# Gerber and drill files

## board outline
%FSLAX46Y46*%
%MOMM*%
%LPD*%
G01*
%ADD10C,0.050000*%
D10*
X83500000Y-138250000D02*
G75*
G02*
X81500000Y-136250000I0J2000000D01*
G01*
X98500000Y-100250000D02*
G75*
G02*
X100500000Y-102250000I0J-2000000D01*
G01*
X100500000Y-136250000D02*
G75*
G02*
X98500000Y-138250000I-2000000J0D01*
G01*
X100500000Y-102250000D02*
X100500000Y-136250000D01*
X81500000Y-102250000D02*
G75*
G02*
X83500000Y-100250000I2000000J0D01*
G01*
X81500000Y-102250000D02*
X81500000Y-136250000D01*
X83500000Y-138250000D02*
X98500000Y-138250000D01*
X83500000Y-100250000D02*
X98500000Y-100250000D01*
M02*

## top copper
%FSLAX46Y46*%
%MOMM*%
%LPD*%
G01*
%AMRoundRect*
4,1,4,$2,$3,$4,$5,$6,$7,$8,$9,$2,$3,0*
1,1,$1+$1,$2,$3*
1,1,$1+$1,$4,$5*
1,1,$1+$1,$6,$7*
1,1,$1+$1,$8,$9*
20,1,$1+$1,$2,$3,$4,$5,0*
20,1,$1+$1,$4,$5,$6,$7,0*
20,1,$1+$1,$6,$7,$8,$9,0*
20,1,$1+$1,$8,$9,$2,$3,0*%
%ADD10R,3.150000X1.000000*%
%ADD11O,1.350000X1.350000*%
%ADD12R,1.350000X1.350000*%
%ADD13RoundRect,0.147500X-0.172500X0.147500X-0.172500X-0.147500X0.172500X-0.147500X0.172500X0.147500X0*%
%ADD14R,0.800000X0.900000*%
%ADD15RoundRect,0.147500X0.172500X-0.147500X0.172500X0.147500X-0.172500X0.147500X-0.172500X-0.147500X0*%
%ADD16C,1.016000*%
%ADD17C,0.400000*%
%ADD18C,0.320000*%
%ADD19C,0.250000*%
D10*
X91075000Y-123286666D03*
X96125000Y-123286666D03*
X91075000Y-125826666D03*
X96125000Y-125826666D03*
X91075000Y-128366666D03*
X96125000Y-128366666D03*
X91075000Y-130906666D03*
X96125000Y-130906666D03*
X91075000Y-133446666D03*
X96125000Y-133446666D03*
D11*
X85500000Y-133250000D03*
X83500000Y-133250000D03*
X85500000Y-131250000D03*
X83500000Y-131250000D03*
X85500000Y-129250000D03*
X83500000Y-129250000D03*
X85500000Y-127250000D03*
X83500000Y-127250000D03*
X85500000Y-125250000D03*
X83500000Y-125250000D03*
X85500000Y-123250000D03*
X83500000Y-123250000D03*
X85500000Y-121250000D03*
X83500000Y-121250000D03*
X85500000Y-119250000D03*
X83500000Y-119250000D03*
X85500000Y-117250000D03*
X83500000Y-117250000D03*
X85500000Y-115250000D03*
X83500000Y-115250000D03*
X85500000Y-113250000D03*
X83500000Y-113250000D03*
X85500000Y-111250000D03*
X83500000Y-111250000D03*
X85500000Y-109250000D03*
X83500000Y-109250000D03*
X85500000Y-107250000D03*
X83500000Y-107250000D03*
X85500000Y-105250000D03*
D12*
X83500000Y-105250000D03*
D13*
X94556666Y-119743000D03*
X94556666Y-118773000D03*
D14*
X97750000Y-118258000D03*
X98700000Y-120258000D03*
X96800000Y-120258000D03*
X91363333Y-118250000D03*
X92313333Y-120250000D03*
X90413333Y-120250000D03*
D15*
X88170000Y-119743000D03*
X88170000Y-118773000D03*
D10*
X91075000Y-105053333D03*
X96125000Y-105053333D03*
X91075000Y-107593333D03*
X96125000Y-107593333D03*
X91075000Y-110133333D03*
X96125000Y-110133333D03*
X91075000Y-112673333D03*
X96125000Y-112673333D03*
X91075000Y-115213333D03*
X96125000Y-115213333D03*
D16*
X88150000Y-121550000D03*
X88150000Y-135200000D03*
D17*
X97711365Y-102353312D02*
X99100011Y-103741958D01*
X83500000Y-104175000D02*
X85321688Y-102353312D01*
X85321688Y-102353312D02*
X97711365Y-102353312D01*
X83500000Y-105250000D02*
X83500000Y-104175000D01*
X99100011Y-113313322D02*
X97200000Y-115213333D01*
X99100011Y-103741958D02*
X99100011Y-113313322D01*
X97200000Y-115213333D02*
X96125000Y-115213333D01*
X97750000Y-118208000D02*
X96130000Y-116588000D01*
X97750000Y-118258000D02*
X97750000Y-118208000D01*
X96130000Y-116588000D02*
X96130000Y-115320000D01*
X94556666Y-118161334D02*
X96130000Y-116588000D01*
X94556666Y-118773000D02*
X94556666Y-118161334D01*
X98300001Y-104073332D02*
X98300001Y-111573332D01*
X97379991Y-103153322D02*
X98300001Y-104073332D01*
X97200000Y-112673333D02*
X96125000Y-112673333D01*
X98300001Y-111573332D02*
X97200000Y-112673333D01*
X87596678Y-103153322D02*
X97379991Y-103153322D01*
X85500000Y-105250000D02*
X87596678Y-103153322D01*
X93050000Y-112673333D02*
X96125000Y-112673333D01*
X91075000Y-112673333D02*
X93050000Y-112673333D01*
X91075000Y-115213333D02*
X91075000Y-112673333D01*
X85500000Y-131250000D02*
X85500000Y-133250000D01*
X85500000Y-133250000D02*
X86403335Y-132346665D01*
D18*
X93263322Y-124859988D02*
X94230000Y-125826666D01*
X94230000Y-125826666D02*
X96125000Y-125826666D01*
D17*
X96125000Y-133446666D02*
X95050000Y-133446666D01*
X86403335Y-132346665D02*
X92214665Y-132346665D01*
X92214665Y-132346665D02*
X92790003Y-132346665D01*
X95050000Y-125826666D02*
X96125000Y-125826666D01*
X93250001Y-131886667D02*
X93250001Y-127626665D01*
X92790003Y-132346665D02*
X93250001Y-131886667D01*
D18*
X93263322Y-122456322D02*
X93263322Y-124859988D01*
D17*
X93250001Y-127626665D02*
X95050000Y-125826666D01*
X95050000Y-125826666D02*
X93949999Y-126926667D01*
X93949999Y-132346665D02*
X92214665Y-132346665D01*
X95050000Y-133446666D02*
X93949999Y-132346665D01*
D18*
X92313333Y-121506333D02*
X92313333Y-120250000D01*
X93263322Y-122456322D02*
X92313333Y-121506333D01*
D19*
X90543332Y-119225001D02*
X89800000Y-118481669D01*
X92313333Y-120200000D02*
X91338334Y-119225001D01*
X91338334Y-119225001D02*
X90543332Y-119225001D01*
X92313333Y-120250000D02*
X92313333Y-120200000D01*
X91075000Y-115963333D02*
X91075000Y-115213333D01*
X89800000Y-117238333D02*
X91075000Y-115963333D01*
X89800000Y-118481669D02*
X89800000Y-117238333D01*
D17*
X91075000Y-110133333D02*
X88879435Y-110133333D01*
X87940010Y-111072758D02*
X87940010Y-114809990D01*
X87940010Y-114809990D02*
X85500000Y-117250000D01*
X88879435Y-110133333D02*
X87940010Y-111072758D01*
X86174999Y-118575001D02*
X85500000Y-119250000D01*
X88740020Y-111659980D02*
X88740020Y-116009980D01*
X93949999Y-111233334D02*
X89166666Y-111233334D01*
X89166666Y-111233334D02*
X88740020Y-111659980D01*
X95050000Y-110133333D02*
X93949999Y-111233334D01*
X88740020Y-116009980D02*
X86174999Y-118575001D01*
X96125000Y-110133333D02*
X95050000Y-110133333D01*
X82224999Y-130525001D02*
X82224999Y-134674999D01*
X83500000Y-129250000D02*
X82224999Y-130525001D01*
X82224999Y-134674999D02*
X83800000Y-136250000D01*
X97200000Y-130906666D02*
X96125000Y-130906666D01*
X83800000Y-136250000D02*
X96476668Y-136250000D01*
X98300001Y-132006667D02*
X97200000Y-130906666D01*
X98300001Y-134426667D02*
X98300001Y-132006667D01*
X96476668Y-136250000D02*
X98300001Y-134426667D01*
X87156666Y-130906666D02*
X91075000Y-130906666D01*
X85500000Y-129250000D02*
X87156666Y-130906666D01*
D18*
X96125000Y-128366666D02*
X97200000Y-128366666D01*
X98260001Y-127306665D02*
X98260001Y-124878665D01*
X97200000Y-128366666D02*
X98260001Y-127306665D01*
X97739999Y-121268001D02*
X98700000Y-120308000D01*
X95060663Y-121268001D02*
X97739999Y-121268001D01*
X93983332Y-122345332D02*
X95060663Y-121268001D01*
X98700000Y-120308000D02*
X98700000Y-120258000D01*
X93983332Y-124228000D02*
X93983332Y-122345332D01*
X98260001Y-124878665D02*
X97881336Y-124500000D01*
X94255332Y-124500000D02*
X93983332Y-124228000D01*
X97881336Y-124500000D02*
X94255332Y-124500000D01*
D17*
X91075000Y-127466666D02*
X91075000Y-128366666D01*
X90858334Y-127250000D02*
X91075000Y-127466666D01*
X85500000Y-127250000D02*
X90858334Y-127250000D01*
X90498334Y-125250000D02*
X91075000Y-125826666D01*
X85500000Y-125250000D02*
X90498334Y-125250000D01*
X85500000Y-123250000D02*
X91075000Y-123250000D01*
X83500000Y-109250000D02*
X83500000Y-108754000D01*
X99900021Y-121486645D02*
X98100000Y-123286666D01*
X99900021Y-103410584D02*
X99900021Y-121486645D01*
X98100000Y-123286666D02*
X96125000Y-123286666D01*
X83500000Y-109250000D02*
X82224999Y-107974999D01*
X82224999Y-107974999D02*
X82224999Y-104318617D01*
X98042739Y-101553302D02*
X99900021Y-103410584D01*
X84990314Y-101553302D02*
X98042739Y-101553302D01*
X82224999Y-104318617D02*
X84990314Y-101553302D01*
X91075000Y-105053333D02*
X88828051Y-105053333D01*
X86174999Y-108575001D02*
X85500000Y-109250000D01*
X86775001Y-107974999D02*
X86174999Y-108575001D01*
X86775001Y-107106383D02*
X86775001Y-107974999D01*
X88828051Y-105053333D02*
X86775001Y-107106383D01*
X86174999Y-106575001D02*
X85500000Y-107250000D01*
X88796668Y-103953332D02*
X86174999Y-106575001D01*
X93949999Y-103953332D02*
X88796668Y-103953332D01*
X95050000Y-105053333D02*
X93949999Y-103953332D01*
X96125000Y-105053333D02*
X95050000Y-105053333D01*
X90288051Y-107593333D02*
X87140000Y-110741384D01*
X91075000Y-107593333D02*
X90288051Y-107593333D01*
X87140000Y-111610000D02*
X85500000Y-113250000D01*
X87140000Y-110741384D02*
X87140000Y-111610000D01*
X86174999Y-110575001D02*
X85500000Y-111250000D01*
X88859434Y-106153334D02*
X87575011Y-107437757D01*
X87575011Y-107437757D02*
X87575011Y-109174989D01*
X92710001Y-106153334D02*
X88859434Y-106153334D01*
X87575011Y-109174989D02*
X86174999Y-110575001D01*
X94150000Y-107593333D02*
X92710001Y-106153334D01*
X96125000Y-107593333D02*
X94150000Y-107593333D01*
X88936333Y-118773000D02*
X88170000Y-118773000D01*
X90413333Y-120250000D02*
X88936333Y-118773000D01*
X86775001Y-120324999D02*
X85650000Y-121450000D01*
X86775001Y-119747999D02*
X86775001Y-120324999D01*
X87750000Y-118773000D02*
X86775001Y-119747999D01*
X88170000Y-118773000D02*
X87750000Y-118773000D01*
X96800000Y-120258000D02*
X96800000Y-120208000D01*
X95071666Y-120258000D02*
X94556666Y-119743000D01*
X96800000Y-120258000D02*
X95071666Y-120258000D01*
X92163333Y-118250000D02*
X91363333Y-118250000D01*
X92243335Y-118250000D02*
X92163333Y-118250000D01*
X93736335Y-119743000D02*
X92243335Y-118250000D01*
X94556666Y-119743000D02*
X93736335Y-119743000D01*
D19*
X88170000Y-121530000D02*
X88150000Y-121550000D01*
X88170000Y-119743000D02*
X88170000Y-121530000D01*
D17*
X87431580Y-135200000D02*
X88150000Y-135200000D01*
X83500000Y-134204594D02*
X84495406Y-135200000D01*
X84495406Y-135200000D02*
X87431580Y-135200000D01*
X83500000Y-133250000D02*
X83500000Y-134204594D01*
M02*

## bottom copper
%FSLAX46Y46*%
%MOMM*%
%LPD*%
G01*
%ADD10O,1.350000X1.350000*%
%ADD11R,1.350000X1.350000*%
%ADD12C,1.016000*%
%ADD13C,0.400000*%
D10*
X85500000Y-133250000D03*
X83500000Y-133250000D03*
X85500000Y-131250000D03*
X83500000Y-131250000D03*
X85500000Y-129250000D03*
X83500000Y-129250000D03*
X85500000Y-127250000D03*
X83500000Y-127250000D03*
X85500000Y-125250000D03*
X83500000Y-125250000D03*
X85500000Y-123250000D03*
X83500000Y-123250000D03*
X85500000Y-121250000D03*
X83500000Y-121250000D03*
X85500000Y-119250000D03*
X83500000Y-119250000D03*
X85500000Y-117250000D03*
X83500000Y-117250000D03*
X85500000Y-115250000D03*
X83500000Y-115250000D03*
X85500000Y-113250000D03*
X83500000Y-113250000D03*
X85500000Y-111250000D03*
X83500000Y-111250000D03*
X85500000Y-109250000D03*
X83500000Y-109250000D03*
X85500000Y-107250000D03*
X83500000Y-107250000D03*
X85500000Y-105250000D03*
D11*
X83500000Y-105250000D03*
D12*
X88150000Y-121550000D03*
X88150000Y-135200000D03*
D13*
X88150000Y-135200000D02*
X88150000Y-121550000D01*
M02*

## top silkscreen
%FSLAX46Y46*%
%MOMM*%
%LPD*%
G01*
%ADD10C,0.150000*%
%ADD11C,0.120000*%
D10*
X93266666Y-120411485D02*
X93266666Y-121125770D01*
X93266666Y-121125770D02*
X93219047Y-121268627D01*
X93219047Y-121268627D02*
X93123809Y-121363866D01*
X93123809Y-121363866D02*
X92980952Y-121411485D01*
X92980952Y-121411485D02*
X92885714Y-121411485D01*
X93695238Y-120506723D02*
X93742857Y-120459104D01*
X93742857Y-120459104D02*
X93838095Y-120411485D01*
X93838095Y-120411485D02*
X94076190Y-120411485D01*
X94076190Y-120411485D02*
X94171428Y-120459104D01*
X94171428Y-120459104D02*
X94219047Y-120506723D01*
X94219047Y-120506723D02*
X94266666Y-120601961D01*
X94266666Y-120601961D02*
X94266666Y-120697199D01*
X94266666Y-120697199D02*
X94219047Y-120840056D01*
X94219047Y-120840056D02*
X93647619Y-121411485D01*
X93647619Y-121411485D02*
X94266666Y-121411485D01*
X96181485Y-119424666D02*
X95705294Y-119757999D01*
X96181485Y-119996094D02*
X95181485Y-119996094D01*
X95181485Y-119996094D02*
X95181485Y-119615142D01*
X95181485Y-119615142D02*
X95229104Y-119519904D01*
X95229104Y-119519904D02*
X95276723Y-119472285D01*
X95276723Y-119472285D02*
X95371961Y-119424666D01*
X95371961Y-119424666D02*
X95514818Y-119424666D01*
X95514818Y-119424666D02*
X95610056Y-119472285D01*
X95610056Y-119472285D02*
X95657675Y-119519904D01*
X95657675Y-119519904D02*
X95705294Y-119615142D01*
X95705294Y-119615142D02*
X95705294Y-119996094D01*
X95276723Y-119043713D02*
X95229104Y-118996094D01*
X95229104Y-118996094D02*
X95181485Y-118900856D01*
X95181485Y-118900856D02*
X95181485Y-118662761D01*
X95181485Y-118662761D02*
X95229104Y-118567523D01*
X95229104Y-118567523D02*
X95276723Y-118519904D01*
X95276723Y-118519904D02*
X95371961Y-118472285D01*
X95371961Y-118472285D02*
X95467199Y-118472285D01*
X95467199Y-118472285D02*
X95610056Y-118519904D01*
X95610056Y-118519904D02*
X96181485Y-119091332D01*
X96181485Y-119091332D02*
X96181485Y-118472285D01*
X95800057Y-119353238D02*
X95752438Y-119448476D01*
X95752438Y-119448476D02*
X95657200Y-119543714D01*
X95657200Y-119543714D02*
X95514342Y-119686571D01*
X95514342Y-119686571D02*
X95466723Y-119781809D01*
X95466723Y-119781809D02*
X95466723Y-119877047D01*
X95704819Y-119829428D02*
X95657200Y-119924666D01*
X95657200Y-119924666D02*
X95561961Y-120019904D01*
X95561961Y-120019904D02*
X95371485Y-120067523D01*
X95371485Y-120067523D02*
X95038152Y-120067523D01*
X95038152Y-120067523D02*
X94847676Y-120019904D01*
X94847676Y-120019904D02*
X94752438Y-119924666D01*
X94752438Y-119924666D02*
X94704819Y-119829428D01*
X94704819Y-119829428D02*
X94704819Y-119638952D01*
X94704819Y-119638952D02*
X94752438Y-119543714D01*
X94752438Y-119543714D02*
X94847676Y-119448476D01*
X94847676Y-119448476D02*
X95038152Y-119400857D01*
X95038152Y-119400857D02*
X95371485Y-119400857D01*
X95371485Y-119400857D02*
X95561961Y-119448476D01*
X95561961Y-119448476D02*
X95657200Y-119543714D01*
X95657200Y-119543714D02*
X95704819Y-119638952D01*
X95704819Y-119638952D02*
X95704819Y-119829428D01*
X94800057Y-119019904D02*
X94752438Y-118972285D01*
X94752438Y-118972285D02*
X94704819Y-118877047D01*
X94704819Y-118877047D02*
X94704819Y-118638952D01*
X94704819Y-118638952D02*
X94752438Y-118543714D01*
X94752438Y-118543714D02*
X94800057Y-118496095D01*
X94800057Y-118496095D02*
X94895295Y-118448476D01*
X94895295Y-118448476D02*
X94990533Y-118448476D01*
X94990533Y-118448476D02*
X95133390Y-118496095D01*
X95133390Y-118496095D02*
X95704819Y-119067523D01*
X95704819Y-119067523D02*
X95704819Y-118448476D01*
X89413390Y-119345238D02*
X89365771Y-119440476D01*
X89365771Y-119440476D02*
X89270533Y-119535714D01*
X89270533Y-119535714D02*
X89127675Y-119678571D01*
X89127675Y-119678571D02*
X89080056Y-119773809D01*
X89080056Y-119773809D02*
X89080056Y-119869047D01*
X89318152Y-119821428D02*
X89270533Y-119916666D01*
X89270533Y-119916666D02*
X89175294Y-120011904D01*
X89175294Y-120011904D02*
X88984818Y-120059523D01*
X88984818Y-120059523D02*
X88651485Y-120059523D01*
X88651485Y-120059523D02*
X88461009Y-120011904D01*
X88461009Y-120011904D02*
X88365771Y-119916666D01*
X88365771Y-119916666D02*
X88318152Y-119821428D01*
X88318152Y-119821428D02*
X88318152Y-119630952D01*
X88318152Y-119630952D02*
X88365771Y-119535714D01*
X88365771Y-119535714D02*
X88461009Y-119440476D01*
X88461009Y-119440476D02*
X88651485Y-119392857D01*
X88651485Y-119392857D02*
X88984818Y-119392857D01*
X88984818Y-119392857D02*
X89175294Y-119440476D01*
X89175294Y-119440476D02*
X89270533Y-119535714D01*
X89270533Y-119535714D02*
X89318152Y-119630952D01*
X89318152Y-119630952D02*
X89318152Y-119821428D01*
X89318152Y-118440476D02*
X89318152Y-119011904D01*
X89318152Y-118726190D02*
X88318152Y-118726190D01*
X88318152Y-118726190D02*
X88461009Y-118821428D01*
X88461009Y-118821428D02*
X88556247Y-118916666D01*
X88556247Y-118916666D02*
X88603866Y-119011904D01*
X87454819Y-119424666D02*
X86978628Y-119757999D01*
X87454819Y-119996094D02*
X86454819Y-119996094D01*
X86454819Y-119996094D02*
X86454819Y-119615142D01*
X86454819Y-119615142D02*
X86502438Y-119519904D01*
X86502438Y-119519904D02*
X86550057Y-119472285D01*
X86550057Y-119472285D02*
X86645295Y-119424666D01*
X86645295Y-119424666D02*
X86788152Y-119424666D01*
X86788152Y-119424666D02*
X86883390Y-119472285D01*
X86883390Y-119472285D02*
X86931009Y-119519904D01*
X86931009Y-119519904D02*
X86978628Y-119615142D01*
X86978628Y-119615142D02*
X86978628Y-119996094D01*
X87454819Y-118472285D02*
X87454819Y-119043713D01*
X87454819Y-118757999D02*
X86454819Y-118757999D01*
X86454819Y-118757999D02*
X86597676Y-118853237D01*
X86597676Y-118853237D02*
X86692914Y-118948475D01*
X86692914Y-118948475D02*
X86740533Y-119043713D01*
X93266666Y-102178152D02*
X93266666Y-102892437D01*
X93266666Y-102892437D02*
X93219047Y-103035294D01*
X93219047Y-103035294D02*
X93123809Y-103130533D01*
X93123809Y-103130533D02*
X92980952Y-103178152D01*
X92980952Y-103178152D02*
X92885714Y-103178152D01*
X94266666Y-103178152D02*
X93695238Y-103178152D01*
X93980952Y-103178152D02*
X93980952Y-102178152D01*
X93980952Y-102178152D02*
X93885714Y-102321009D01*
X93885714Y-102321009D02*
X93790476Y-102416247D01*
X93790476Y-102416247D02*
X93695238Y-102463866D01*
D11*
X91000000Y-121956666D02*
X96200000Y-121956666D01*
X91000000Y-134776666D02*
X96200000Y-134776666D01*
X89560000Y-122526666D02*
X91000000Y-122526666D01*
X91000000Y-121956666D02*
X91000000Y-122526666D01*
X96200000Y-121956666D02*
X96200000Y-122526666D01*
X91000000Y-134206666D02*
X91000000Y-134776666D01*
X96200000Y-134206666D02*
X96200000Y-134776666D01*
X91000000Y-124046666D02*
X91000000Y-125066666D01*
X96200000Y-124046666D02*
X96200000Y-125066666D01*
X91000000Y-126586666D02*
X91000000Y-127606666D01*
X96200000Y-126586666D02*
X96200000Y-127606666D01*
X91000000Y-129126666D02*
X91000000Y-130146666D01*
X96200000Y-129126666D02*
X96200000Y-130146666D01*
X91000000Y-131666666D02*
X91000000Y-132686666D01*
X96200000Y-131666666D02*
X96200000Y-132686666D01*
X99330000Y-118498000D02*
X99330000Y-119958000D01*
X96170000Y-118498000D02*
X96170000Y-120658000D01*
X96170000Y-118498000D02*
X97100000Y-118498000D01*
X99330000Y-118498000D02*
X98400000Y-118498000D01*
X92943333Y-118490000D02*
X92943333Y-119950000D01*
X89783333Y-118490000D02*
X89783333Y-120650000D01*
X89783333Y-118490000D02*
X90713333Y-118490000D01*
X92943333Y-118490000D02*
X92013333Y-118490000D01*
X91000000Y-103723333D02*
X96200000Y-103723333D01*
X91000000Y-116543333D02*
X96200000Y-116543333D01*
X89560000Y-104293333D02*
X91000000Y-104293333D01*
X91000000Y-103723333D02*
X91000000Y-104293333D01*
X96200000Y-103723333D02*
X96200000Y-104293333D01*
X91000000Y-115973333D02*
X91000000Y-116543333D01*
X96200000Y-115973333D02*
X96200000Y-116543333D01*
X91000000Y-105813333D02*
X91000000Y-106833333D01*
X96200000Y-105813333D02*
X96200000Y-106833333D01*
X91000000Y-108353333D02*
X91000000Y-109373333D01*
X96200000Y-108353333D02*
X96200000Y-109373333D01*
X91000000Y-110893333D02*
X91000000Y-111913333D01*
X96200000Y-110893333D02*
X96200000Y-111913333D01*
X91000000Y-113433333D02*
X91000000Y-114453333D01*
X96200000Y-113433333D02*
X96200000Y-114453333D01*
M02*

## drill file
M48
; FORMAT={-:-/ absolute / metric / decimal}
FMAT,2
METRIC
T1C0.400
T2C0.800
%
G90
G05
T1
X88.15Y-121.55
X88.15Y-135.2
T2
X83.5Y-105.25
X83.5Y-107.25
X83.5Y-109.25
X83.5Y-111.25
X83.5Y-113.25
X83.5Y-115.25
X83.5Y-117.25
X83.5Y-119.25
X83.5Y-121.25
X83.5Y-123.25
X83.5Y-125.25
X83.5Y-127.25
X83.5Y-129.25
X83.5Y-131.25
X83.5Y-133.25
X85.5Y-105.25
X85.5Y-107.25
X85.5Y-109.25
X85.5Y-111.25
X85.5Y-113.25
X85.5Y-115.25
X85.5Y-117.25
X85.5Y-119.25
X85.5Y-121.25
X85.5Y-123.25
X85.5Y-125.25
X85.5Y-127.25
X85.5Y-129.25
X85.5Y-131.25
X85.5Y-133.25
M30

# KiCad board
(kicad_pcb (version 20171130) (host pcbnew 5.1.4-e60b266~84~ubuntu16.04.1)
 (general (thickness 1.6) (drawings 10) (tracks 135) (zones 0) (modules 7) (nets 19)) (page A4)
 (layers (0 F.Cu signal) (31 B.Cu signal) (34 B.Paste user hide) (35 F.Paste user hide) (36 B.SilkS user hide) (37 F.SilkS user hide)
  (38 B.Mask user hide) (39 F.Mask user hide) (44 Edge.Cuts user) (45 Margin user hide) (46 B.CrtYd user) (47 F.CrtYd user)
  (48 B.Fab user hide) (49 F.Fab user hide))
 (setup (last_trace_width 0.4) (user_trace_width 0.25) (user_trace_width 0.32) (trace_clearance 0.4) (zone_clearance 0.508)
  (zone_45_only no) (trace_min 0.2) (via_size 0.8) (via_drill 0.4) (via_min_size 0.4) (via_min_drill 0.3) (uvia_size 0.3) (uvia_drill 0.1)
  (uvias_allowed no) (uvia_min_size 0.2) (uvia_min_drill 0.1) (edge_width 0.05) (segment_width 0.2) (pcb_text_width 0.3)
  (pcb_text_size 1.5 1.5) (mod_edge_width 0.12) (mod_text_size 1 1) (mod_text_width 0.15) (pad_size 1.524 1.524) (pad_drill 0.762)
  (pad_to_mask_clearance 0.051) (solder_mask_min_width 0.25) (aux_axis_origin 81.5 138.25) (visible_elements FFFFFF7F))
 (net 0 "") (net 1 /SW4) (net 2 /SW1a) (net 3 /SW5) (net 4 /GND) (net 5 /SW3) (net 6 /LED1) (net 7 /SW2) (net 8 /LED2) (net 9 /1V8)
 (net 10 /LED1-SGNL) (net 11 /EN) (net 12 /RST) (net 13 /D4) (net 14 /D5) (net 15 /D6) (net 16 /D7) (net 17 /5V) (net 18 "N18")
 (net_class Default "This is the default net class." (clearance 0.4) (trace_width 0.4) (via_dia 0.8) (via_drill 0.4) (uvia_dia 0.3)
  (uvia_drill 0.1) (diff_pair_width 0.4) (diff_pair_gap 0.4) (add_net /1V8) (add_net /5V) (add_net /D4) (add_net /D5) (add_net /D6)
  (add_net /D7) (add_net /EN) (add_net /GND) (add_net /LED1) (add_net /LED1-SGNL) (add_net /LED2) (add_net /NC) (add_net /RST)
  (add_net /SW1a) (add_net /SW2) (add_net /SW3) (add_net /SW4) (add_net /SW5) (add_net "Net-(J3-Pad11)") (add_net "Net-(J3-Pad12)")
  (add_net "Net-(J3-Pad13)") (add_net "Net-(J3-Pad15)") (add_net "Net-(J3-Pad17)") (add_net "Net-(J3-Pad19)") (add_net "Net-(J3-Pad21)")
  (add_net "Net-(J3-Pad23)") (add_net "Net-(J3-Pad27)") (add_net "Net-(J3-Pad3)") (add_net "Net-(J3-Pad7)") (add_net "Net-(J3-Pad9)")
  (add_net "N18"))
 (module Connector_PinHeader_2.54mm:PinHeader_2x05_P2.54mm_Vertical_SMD (layer F.Cu) (at 93.6 128.366666)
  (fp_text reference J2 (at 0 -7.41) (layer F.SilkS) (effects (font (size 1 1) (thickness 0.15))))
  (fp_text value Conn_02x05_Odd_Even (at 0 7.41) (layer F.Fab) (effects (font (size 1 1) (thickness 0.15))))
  (fp_line (start -2.6 -6.41) (end 2.6 -6.41) (layer F.SilkS) (width 0.12))
  (fp_line (start -2.6 6.41) (end 2.6 6.41) (layer F.SilkS) (width 0.12))
  (fp_line (start -4.04 -5.84) (end -2.6 -5.84) (layer F.SilkS) (width 0.12))
  (fp_line (start -2.6 -6.41) (end -2.6 -5.84) (layer F.SilkS) (width 0.12))
  (fp_line (start 2.6 -6.41) (end 2.6 -5.84) (layer F.SilkS) (width 0.12))
  (fp_line (start -2.6 5.84) (end -2.6 6.41) (layer F.SilkS) (width 0.12))
  (fp_line (start 2.6 5.84) (end 2.6 6.41) (layer F.SilkS) (width 0.12))
  (fp_line (start -2.6 -4.32) (end -2.6 -3.3) (layer F.SilkS) (width 0.12))
  (fp_line (start 2.6 -4.32) (end 2.6 -3.3) (layer F.SilkS) (width 0.12))
  (fp_line (start -2.6 -1.78) (end -2.6 -0.76) (layer F.SilkS) (width 0.12))
  (fp_line (start 2.6 -1.78) (end 2.6 -0.76) (layer F.SilkS) (width 0.12))
  (fp_line (start -2.6 0.76) (end -2.6 1.78) (layer F.SilkS) (width 0.12))
  (fp_line (start 2.6 0.76) (end 2.6 1.78) (layer F.SilkS) (width 0.12))
  (fp_line (start -2.6 3.3) (end -2.6 4.32) (layer F.SilkS) (width 0.12))
  (fp_line (start 2.6 3.3) (end 2.6 4.32) (layer F.SilkS) (width 0.12))
  (pad 1 smd rect (at -2.525 -5.08) (size 3.15 1) (layers F.Cu F.Paste F.Mask) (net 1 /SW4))
  (pad 2 smd rect (at 2.525 -5.08) (size 3.15 1) (layers F.Cu F.Paste F.Mask) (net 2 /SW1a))
  (pad 3 smd rect (at -2.525 -2.54) (size 3.15 1) (layers F.Cu F.Paste F.Mask) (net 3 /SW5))
  (pad 4 smd rect (at 2.525 -2.54) (size 3.15 1) (layers F.Cu F.Paste F.Mask) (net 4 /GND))
  (pad 5 smd rect (at -2.525 0) (size 3.15 1) (layers F.Cu F.Paste F.Mask) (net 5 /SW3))
  (pad 6 smd rect (at 2.525 0) (size 3.15 1) (layers F.Cu F.Paste F.Mask) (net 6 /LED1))
  (pad 7 smd rect (at -2.525 2.54) (size 3.15 1) (layers F.Cu F.Paste F.Mask) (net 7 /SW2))
  (pad 8 smd rect (at 2.525 2.54) (size 3.15 1) (layers F.Cu F.Paste F.Mask) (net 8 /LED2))
  (pad 9 smd rect (at -2.525 5.08) (size 3.15 1) (layers F.Cu F.Paste F.Mask))
  (pad 10 smd rect (at 2.525 5.08) (size 3.15 1) (layers F.Cu F.Paste F.Mask) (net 4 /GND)))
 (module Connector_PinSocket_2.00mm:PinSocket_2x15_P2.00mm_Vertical (layer B.Cu) (at 83.5 105.25 180)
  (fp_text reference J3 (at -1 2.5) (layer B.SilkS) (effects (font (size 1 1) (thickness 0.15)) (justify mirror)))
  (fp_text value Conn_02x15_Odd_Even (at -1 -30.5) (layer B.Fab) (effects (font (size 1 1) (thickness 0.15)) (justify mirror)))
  (pad 30 thru_hole oval (at -2 -28 180) (size 1.35 1.35) (drill 0.8) (layers *.Cu *.Mask) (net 4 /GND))
  (pad 29 thru_hole oval (at 0 -28 180) (size 1.35 1.35) (drill 0.8) (layers *.Cu *.Mask) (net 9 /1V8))
  (pad 28 thru_hole oval (at -2 -26 180) (size 1.35 1.35) (drill 0.8) (layers *.Cu *.Mask) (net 4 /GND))
  (pad 27 thru_hole oval (at 0 -26 180) (size 1.35 1.35) (drill 0.8) (layers *.Cu *.Mask))
  (pad 26 thru_hole oval (at -2 -24 180) (size 1.35 1.35) (drill 0.8) (layers *.Cu *.Mask) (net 7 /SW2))
  (pad 25 thru_hole oval (at 0 -24 180) (size 1.35 1.35) (drill 0.8) (layers *.Cu *.Mask) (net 8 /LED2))
  (pad 24 thru_hole oval (at -2 -22 180) (size 1.35 1.35) (drill 0.8) (layers *.Cu *.Mask) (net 5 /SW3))
  (pad 23 thru_hole oval (at 0 -22 180) (size 1.35 1.35) (drill 0.8) (layers *.Cu *.Mask))
  (pad 22 thru_hole oval (at -2 -20 180) (size 1.35 1.35) (drill 0.8) (layers *.Cu *.Mask) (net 3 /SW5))
  (pad 21 thru_hole oval (at 0 -20 180) (size 1.35 1.35) (drill 0.8) (layers *.Cu *.Mask))
  (pad 20 thru_hole oval (at -2 -18 180) (size 1.35 1.35) (drill 0.8) (layers *.Cu *.Mask) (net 1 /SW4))
  (pad 19 thru_hole oval (at 0 -18 180) (size 1.35 1.35) (drill 0.8) (layers *.Cu *.Mask))
  (pad 18 thru_hole oval (at -2 -16 180) (size 1.35 1.35) (drill 0.8) (layers *.Cu *.Mask) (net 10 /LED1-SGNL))
  (pad 17 thru_hole oval (at 0 -16 180) (size 1.35 1.35) (drill 0.8) (layers *.Cu *.Mask))
  (pad 16 thru_hole oval (at -2 -14 180) (size 1.35 1.35) (drill 0.8) (layers *.Cu *.Mask) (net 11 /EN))
  (pad 15 thru_hole oval (at 0 -14 180) (size 1.35 1.35) (drill 0.8) (layers *.Cu *.Mask))
  (pad 14 thru_hole oval (at -2 -12 180) (size 1.35 1.35) (drill 0.8) (layers *.Cu *.Mask) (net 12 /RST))
  (pad 13 thru_hole oval (at 0 -12 180) (size 1.35 1.35) (drill 0.8) (layers *.Cu *.Mask))
  (pad 12 thru_hole oval (at -2 -10 180) (size 1.35 1.35) (drill 0.8) (layers *.Cu *.Mask))
  (pad 11 thru_hole oval (at 0 -10 180) (size 1.35 1.35) (drill 0.8) (layers *.Cu *.Mask))
  (pad 10 thru_hole oval (at -2 -8 180) (size 1.35 1.35) (drill 0.8) (layers *.Cu *.Mask) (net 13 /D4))
  (pad 9 thru_hole oval (at 0 -8 180) (size 1.35 1.35) (drill 0.8) (layers *.Cu *.Mask))
  (pad 8 thru_hole oval (at -2 -6 180) (size 1.35 1.35) (drill 0.8) (layers *.Cu *.Mask) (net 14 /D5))
  (pad 7 thru_hole oval (at 0 -6 180) (size 1.35 1.35) (drill 0.8) (layers *.Cu *.Mask))
  (pad 6 thru_hole oval (at -2 -4 180) (size 1.35 1.35) (drill 0.8) (layers *.Cu *.Mask) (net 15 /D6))
  (pad 5 thru_hole oval (at 0 -4 180) (size 1.35 1.35) (drill 0.8) (layers *.Cu *.Mask) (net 2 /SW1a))
  (pad 4 thru_hole oval (at -2 -2 180) (size 1.35 1.35) (drill 0.8) (layers *.Cu *.Mask) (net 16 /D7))
  (pad 3 thru_hole oval (at 0 -2 180) (size 1.35 1.35) (drill 0.8) (layers *.Cu *.Mask))
  (pad 2 thru_hole oval (at -2 0 180) (size 1.35 1.35) (drill 0.8) (layers *.Cu *.Mask) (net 4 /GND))
  (pad 1 thru_hole rect (at 0 0 180) (size 1.35 1.35) (drill 0.8) (layers *.Cu *.Mask) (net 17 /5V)))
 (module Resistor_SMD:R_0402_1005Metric (layer F.Cu) (at 94.556666 119.258 270)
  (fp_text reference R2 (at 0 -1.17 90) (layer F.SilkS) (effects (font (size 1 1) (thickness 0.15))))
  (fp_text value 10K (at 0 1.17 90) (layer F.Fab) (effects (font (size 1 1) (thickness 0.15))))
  (pad 2 smd roundrect (at 0.485 0 270) (size 0.59 0.64) (layers F.Cu F.Paste F.Mask) (roundrect_rratio 0.25) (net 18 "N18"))
  (pad 1 smd roundrect (at -0.485 0 270) (size 0.59 0.64) (layers F.Cu F.Paste F.Mask) (roundrect_rratio 0.25) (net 17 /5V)))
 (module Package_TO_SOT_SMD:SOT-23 (layer F.Cu) (at 97.75 119.258 90)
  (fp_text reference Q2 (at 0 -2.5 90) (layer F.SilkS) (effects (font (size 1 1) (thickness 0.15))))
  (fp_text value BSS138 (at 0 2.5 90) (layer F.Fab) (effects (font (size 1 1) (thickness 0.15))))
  (fp_line (start 0.76 1.58) (end -0.7 1.58) (layer F.SilkS) (width 0.12))
  (fp_line (start 0.76 -1.58) (end -1.4 -1.58) (layer F.SilkS) (width 0.12))
  (fp_line (start 0.76 -1.58) (end 0.76 -0.65) (layer F.SilkS) (width 0.12))
  (fp_line (start 0.76 1.58) (end 0.76 0.65) (layer F.SilkS) (width 0.12))
  (pad 3 smd rect (at 1 0 90) (size 0.9 0.8) (layers F.Cu F.Paste F.Mask) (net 17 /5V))
  (pad 2 smd rect (at -1 0.95 90) (size 0.9 0.8) (layers F.Cu F.Paste F.Mask) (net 6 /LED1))
  (pad 1 smd rect (at -1 -0.95 90) (size 0.9 0.8) (layers F.Cu F.Paste F.Mask) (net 18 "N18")))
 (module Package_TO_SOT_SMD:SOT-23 (layer F.Cu) (at 91.363333 119.25 90)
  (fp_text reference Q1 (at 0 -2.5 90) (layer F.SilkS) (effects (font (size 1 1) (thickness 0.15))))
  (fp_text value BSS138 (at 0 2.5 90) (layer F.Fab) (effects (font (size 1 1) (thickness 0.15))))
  (fp_line (start 0.76 1.58) (end -0.7 1.58) (layer F.SilkS) (width 0.12))
  (fp_line (start 0.76 -1.58) (end -1.4 -1.58) (layer F.SilkS) (width 0.12))
  (fp_line (start 0.76 -1.58) (end 0.76 -0.65) (layer F.SilkS) (width 0.12))
  (fp_line (start 0.76 1.58) (end 0.76 0.65) (layer F.SilkS) (width 0.12))
  (pad 3 smd rect (at 1 0 90) (size 0.9 0.8) (layers F.Cu F.Paste F.Mask) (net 18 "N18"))
  (pad 2 smd rect (at -1 0.95 90) (size 0.9 0.8) (layers F.Cu F.Paste F.Mask) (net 4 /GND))
  (pad 1 smd rect (at -1 -0.95 90) (size 0.9 0.8) (layers F.Cu F.Paste F.Mask) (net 10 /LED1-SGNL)))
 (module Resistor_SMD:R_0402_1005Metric (layer F.Cu) (at 88.17 119.258 90)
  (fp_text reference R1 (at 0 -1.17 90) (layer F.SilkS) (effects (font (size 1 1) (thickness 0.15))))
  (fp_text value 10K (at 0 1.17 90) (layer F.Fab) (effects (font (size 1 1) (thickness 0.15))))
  (pad 1 smd roundrect (at -0.485 0 90) (size 0.59 0.64) (layers F.Cu F.Paste F.Mask) (roundrect_rratio 0.25) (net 9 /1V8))
  (pad 2 smd roundrect (at 0.485 0 90) (size 0.59 0.64) (layers F.Cu F.Paste F.Mask) (roundrect_rratio 0.25) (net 10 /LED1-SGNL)))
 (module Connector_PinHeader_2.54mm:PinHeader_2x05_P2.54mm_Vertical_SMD (layer F.Cu) (at 93.6 110.133333)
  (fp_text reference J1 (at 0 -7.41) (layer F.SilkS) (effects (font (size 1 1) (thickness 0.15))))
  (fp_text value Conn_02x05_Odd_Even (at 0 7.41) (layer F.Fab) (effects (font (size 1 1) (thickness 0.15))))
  (fp_line (start -2.6 -6.41) (end 2.6 -6.41) (layer F.SilkS) (width 0.12))
  (fp_line (start -2.6 6.41) (end 2.6 6.41) (layer F.SilkS) (width 0.12))
  (fp_line (start -4.04 -5.84) (end -2.6 -5.84) (layer F.SilkS) (width 0.12))
  (fp_line (start -2.6 -6.41) (end -2.6 -5.84) (layer F.SilkS) (width 0.12))
  (fp_line (start 2.6 -6.41) (end 2.6 -5.84) (layer F.SilkS) (width 0.12))
  (fp_line (start -2.6 5.84) (end -2.6 6.41) (layer F.SilkS) (width 0.12))
  (fp_line (start 2.6 5.84) (end 2.6 6.41) (layer F.SilkS) (width 0.12))
  (fp_line (start -2.6 -4.32) (end -2.6 -3.3) (layer F.SilkS) (width 0.12))
  (fp_line (start 2.6 -4.32) (end 2.6 -3.3) (layer F.SilkS) (width 0.12))
  (fp_line (start -2.6 -1.78) (end -2.6 -0.76) (layer F.SilkS) (width 0.12))
  (fp_line (start 2.6 -1.78) (end 2.6 -0.76) (layer F.SilkS) (width 0.12))
  (fp_line (start -2.6 0.76) (end -2.6 1.78) (layer F.SilkS) (width 0.12))
  (fp_line (start 2.6 0.76) (end 2.6 1.78) (layer F.SilkS) (width 0.12))
  (fp_line (start -2.6 3.3) (end -2.6 4.32) (layer F.SilkS) (width 0.12))
  (fp_line (start 2.6 3.3) (end 2.6 4.32) (layer F.SilkS) (width 0.12))
  (pad 1 smd rect (at -2.525 -5.08) (size 3.15 1) (layers F.Cu F.Paste F.Mask) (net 15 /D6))
  (pad 2 smd rect (at 2.525 -5.08) (size 3.15 1) (layers F.Cu F.Paste F.Mask) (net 16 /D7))
  (pad 3 smd rect (at -2.525 -2.54) (size 3.15 1) (layers F.Cu F.Paste F.Mask) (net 13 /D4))
  (pad 4 smd rect (at 2.525 -2.54) (size 3.15 1) (layers F.Cu F.Paste F.Mask) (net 14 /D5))
  (pad 5 smd rect (at -2.525 0) (size 3.15 1) (layers F.Cu F.Paste F.Mask) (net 12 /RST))
  (pad 6 smd rect (at 2.525 0) (size 3.15 1) (layers F.Cu F.Paste F.Mask) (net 11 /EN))
  (pad 7 smd rect (at -2.525 2.54) (size 3.15 1) (layers F.Cu F.Paste F.Mask) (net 4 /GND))
  (pad 8 smd rect (at 2.525 2.54) (size 3.15 1) (layers F.Cu F.Paste F.Mask) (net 4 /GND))
  (pad 9 smd rect (at -2.525 5.08) (size 3.15 1) (layers F.Cu F.Paste F.Mask) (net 4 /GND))
  (pad 10 smd rect (at 2.525 5.08) (size 3.15 1) (layers F.Cu F.Paste F.Mask) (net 17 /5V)))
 (gr_arc (start 83.5 136.25) (end 81.5 136.25) (angle -90) (layer Edge.Cuts) (width 0.05))
 (gr_arc (start 98.5 102.25) (end 100.5 102.25) (angle -90) (layer Edge.Cuts) (width 0.05))
 (gr_arc (start 98.5 136.25) (end 98.5 138.25) (angle -90) (layer Edge.Cuts) (width 0.05))
 (gr_line (start 100.5 102.25) (end 100.5 136.25) (layer Edge.Cuts) (width 0.05))
 (gr_arc (start 83.5 102.25) (end 83.5 100.25) (angle -90) (layer Edge.Cuts) (width 0.05))
 (gr_line (start 81.5 102.25) (end 81.5 136.25) (layer Edge.Cuts) (width 0.05))
 (gr_line (start 83.5 138.25) (end 98.5 138.25) (layer Edge.Cuts) (width 0.05))
 (gr_line (start 83.5 100.25) (end 98.5 100.25) (layer Edge.Cuts) (width 0.05))
 (via (at 88.15 121.55) (size 1.016) (drill 0.4) (layers F.Cu B.Cu) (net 9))
 (via (at 88.15 135.2) (size 1.016) (drill 0.4) (layers F.Cu B.Cu) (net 9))
 (segment (start 97.711365 102.353312) (end 99.100011 103.741958) (width 0.4) (layer F.Cu) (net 17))
 (segment (start 83.5 104.175) (end 85.321688 102.353312) (width 0.4) (layer F.Cu) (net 17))
 (segment (start 85.321688 102.353312) (end 97.711365 102.353312) (width 0.4) (layer F.Cu) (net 17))
 (segment (start 83.5 105.25) (end 83.5 104.175) (width 0.4) (layer F.Cu) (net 17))
 (segment (start 99.100011 113.313322) (end 97.2 115.213333) (width 0.4) (layer F.Cu) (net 17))
 (segment (start 99.100011 103.741958) (end 99.100011 113.313322) (width 0.4) (layer F.Cu) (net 17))
 (segment (start 97.2 115.213333) (end 96.125 115.213333) (width 0.4) (layer F.Cu) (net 17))
 (segment (start 97.75 118.208) (end 96.13 116.588) (width 0.4) (layer F.Cu) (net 17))
 (segment (start 97.75 118.258) (end 97.75 118.208) (width 0.4) (layer F.Cu) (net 17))
 (segment (start 96.13 116.588) (end 96.13 115.32) (width 0.4) (layer F.Cu) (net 17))
 (segment (start 94.556666 118.161334) (end 96.13 116.588) (width 0.4) (layer F.Cu) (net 17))
 (segment (start 94.556666 118.773) (end 94.556666 118.161334) (width 0.4) (layer F.Cu) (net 17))
 (segment (start 98.300001 104.073332) (end 98.300001 111.573332) (width 0.4) (layer F.Cu) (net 4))
 (segment (start 97.379991 103.153322) (end 98.300001 104.073332) (width 0.4) (layer F.Cu) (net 4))
 (segment (start 97.2 112.673333) (end 96.125 112.673333) (width 0.4) (layer F.Cu) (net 4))
 (segment (start 98.300001 111.573332) (end 97.2 112.673333) (width 0.4) (layer F.Cu) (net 4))
 (segment (start 87.596678 103.153322) (end 97.379991 103.153322) (width 0.4) (layer F.Cu) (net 4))
 (segment (start 85.5 105.25) (end 87.596678 103.153322) (width 0.4) (layer F.Cu) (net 4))
 (segment (start 93.05 112.673333) (end 96.125 112.673333) (width 0.4) (layer F.Cu) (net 4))
 (segment (start 91.075 112.673333) (end 93.05 112.673333) (width 0.4) (layer F.Cu) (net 4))
 (segment (start 91.075 115.213333) (end 91.075 112.673333) (width 0.4) (layer F.Cu) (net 4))
 (segment (start 85.5 131.25) (end 85.5 133.25) (width 0.4) (layer F.Cu) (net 4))
 (segment (start 85.5 133.25) (end 86.403335 132.346665) (width 0.4) (layer F.Cu) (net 4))
 (segment (start 93.263322 124.859988) (end 94.23 125.826666) (width 0.32) (layer F.Cu) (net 4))
 (segment (start 94.23 125.826666) (end 96.125 125.826666) (width 0.32) (layer F.Cu) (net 4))
 (segment (start 96.125 133.446666) (end 95.05 133.446666) (width 0.4) (layer F.Cu) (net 4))
 (segment (start 86.403335 132.346665) (end 92.214665 132.346665) (width 0.4) (layer F.Cu) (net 4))
 (segment (start 92.214665 132.346665) (end 92.790003 132.346665) (width 0.4) (layer F.Cu) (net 4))
 (segment (start 95.05 125.826666) (end 96.125 125.826666) (width 0.4) (layer F.Cu) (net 4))
 (segment (start 93.250001 131.886667) (end 93.250001 127.626665) (width 0.4) (layer F.Cu) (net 4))
 (segment (start 92.790003 132.346665) (end 93.250001 131.886667) (width 0.4) (layer F.Cu) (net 4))
 (segment (start 93.263322 122.456322) (end 93.263322 124.859988) (width 0.32) (layer F.Cu) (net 4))
 (segment (start 93.250001 127.626665) (end 95.05 125.826666) (width 0.4) (layer F.Cu) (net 4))
 (segment (start 95.05 125.826666) (end 93.949999 126.926667) (width 0.4) (layer F.Cu) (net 4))
 (segment (start 93.949999 132.346665) (end 92.214665 132.346665) (width 0.4) (layer F.Cu) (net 4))
 (segment (start 95.05 133.446666) (end 93.949999 132.346665) (width 0.4) (layer F.Cu) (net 4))
 (segment (start 92.313333 121.506333) (end 92.313333 120.25) (width 0.32) (layer F.Cu) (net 4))
 (segment (start 93.263322 122.456322) (end 92.313333 121.506333) (width 0.32) (layer F.Cu) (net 4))
 (segment (start 90.543332 119.225001) (end 89.8 118.481669) (width 0.25) (layer F.Cu) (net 4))
 (segment (start 92.313333 120.2) (end 91.338334 119.225001) (width 0.25) (layer F.Cu) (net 4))
 (segment (start 91.338334 119.225001) (end 90.543332 119.225001) (width 0.25) (layer F.Cu) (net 4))
 (segment (start 92.313333 120.25) (end 92.313333 120.2) (width 0.25) (layer F.Cu) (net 4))
 (segment (start 91.075 115.963333) (end 91.075 115.213333) (width 0.25) (layer F.Cu) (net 4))
 (segment (start 89.8 117.238333) (end 91.075 115.963333) (width 0.25) (layer F.Cu) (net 4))
 (segment (start 89.8 118.481669) (end 89.8 117.238333) (width 0.25) (layer F.Cu) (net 4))
 (segment (start 91.075 110.133333) (end 88.879435 110.133333) (width 0.4) (layer F.Cu) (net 12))
 (segment (start 87.94001 111.072758) (end 87.94001 114.80999) (width 0.4) (layer F.Cu) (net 12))
 (segment (start 87.94001 114.80999) (end 85.5 117.25) (width 0.4) (layer F.Cu) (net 12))
 (segment (start 88.879435 110.133333) (end 87.94001 111.072758) (width 0.4) (layer F.Cu) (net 12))
 (segment (start 86.174999 118.575001) (end 85.5 119.25) (width 0.4) (layer F.Cu) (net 11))
 (segment (start 88.74002 111.65998) (end 88.74002 116.00998) (width 0.4) (layer F.Cu) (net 11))
 (segment (start 93.949999 111.233334) (end 89.166666 111.233334) (width 0.4) (layer F.Cu) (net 11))
 (segment (start 89.166666 111.233334) (end 88.74002 111.65998) (width 0.4) (layer F.Cu) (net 11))
 (segment (start 95.05 110.133333) (end 93.949999 111.233334) (width 0.4) (layer F.Cu) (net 11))
 (segment (start 88.74002 116.00998) (end 86.174999 118.575001) (width 0.4) (layer F.Cu) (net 11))
 (segment (start 96.125 110.133333) (end 95.05 110.133333) (width 0.4) (layer F.Cu) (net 11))
 (segment (start 82.224999 130.525001) (end 82.224999 134.674999) (width 0.4) (layer F.Cu) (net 8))
 (segment (start 83.5 129.25) (end 82.224999 130.525001) (width 0.4) (layer F.Cu) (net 8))
 (segment (start 82.224999 134.674999) (end 83.8 136.25) (width 0.4) (layer F.Cu) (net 8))
 (segment (start 97.2 130.906666) (end 96.125 130.906666) (width 0.4) (layer F.Cu) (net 8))
 (segment (start 83.8 136.25) (end 96.476668 136.25) (width 0.4) (layer F.Cu) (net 8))
 (segment (start 98.300001 132.006667) (end 97.2 130.906666) (width 0.4) (layer F.Cu) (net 8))
 (segment (start 98.300001 134.426667) (end 98.300001 132.006667) (width 0.4) (layer F.Cu) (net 8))
 (segment (start 96.476668 136.25) (end 98.300001 134.426667) (width 0.4) (layer F.Cu) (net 8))
 (segment (start 87.156666 130.906666) (end 91.075 130.906666) (width 0.4) (layer F.Cu) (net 7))
 (segment (start 85.5 129.25) (end 87.156666 130.906666) (width 0.4) (layer F.Cu) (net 7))
 (segment (start 96.125 128.366666) (end 97.2 128.366666) (width 0.32) (layer F.Cu) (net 6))
 (segment (start 98.260001 127.306665) (end 98.260001 124.878665) (width 0.32) (layer F.Cu) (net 6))
 (segment (start 97.2 128.366666) (end 98.260001 127.306665) (width 0.32) (layer F.Cu) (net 6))
 (segment (start 97.739999 121.268001) (end 98.7 120.308) (width 0.32) (layer F.Cu) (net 6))
 (segment (start 95.060663 121.268001) (end 97.739999 121.268001) (width 0.32) (layer F.Cu) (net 6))
 (segment (start 93.983332 122.345332) (end 95.060663 121.268001) (width 0.32) (layer F.Cu) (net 6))
 (segment (start 98.7 120.308) (end 98.7 120.258) (width 0.32) (layer F.Cu) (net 6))
 (segment (start 93.983332 124.228) (end 93.983332 122.345332) (width 0.32) (layer F.Cu) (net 6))
 (segment (start 98.260001 124.878665) (end 97.881336 124.5) (width 0.32) (layer F.Cu) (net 6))
 (segment (start 94.255332 124.5) (end 93.983332 124.228) (width 0.32) (layer F.Cu) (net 6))
 (segment (start 97.881336 124.5) (end 94.255332 124.5) (width 0.32) (layer F.Cu) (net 6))
 (segment (start 91.075 127.466666) (end 91.075 128.366666) (width 0.4) (layer F.Cu) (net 5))
 (segment (start 90.858334 127.25) (end 91.075 127.466666) (width 0.4) (layer F.Cu) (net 5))
 (segment (start 85.5 127.25) (end 90.858334 127.25) (width 0.4) (layer F.Cu) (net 5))
 (segment (start 90.498334 125.25) (end 91.075 125.826666) (width 0.4) (layer F.Cu) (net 3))
 (segment (start 85.5 125.25) (end 90.498334 125.25) (width 0.4) (layer F.Cu) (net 3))
 (segment (start 85.5 123.25) (end 91.075 123.25) (width 0.4) (layer F.Cu) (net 1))
 (segment (start 83.5 109.25) (end 83.5 108.754) (width 0.4) (layer F.Cu) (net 2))
 (segment (start 99.900021 121.486645) (end 98.1 123.286666) (width 0.4) (layer F.Cu) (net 2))
 (segment (start 99.900021 103.410584) (end 99.900021 121.486645) (width 0.4) (layer F.Cu) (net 2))
 (segment (start 98.1 123.286666) (end 96.125 123.286666) (width 0.4) (layer F.Cu) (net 2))
 (segment (start 83.5 109.25) (end 82.224999 107.974999) (width 0.4) (layer F.Cu) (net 2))
 (segment (start 82.224999 107.974999) (end 82.224999 104.318617) (width 0.4) (layer F.Cu) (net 2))
 (segment (start 98.042739 101.553302) (end 99.900021 103.410584) (width 0.4) (layer F.Cu) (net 2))
 (segment (start 84.990314 101.553302) (end 98.042739 101.553302) (width 0.4) (layer F.Cu) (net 2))
 (segment (start 82.224999 104.318617) (end 84.990314 101.553302) (width 0.4) (layer F.Cu) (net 2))
 (segment (start 91.075 105.053333) (end 88.828051 105.053333) (width 0.4) (layer F.Cu) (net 15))
 (segment (start 86.174999 108.575001) (end 85.5 109.25) (width 0.4) (layer F.Cu) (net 15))
 (segment (start 86.775001 107.974999) (end 86.174999 108.575001) (width 0.4) (layer F.Cu) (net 15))
 (segment (start 86.775001 107.106383) (end 86.775001 107.974999) (width 0.4) (layer F.Cu) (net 15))
 (segment (start 88.828051 105.053333) (end 86.775001 107.106383) (width 0.4) (layer F.Cu) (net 15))
 (segment (start 86.174999 106.575001) (end 85.5 107.25) (width 0.4) (layer F.Cu) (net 16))
 (segment (start 88.796668 103.953332) (end 86.174999 106.575001) (width 0.4) (layer F.Cu) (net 16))
 (segment (start 93.949999 103.953332) (end 88.796668 103.953332) (width 0.4) (layer F.Cu) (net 16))
 (segment (start 95.05 105.053333) (end 93.949999 103.953332) (width 0.4) (layer F.Cu) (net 16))
 (segment (start 96.125 105.053333) (end 95.05 105.053333) (width 0.4) (layer F.Cu) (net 16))
 (segment (start 90.288051 107.593333) (end 87.14 110.741384) (width 0.4) (layer F.Cu) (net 13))
 (segment (start 91.075 107.593333) (end 90.288051 107.593333) (width 0.4) (layer F.Cu) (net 13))
 (segment (start 87.14 111.61) (end 85.5 113.25) (width 0.4) (layer F.Cu) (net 13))
 (segment (start 87.14 110.741384) (end 87.14 111.61) (width 0.4) (layer F.Cu) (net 13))
 (segment (start 86.174999 110.575001) (end 85.5 111.25) (width 0.4) (layer F.Cu) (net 14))
 (segment (start 88.859434 106.153334) (end 87.575011 107.437757) (width 0.4) (layer F.Cu) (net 14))
 (segment (start 87.575011 107.437757) (end 87.575011 109.174989) (width 0.4) (layer F.Cu) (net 14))
 (segment (start 92.710001 106.153334) (end 88.859434 106.153334) (width 0.4) (layer F.Cu) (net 14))
 (segment (start 87.575011 109.174989) (end 86.174999 110.575001) (width 0.4) (layer F.Cu) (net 14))
 (segment (start 94.15 107.593333) (end 92.710001 106.153334) (width 0.4) (layer F.Cu) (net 14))
 (segment (start 96.125 107.593333) (end 94.15 107.593333) (width 0.4) (layer F.Cu) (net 14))
 (segment (start 88.936333 118.773) (end 88.17 118.773) (width 0.4) (layer F.Cu) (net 10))
 (segment (start 90.413333 120.25) (end 88.936333 118.773) (width 0.4) (layer F.Cu) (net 10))
 (segment (start 86.775001 120.324999) (end 85.65 121.45) (width 0.4) (layer F.Cu) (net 10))
 (segment (start 86.775001 119.747999) (end 86.775001 120.324999) (width 0.4) (layer F.Cu) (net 10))
 (segment (start 87.75 118.773) (end 86.775001 119.747999) (width 0.4) (layer F.Cu) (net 10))
 (segment (start 88.17 118.773) (end 87.75 118.773) (width 0.4) (layer F.Cu) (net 10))
 (segment (start 96.8 120.258) (end 96.8 120.208) (width 0.4) (layer F.Cu) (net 18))
 (segment (start 95.071666 120.258) (end 94.556666 119.743) (width 0.4) (layer F.Cu) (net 18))
 (segment (start 96.8 120.258) (end 95.071666 120.258) (width 0.4) (layer F.Cu) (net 18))
 (segment (start 92.163333 118.25) (end 91.363333 118.25) (width 0.4) (layer F.Cu) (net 18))
 (segment (start 92.243335 118.25) (end 92.163333 118.25) (width 0.4) (layer F.Cu) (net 18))
 (segment (start 93.736335 119.743) (end 92.243335 118.25) (width 0.4) (layer F.Cu) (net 18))
 (segment (start 94.556666 119.743) (end 93.736335 119.743) (width 0.4) (layer F.Cu) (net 18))
 (segment (start 88.17 121.53) (end 88.15 121.55) (width 0.25) (layer F.Cu) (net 9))
 (segment (start 88.17 119.743) (end 88.17 121.53) (width 0.25) (layer F.Cu) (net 9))
 (segment (start 87.43158 135.2) (end 88.15 135.2) (width 0.4) (layer F.Cu) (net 9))
 (segment (start 83.5 134.204594) (end 84.495406 135.2) (width 0.4) (layer F.Cu) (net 9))
 (segment (start 84.495406 135.2) (end 87.43158 135.2) (width 0.4) (layer F.Cu) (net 9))
 (segment (start 83.5 133.25) (end 83.5 134.204594) (width 0.4) (layer F.Cu) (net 9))
 (segment (start 88.15 135.2) (end 88.15 121.55) (width 0.4) (layer B.Cu) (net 9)))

